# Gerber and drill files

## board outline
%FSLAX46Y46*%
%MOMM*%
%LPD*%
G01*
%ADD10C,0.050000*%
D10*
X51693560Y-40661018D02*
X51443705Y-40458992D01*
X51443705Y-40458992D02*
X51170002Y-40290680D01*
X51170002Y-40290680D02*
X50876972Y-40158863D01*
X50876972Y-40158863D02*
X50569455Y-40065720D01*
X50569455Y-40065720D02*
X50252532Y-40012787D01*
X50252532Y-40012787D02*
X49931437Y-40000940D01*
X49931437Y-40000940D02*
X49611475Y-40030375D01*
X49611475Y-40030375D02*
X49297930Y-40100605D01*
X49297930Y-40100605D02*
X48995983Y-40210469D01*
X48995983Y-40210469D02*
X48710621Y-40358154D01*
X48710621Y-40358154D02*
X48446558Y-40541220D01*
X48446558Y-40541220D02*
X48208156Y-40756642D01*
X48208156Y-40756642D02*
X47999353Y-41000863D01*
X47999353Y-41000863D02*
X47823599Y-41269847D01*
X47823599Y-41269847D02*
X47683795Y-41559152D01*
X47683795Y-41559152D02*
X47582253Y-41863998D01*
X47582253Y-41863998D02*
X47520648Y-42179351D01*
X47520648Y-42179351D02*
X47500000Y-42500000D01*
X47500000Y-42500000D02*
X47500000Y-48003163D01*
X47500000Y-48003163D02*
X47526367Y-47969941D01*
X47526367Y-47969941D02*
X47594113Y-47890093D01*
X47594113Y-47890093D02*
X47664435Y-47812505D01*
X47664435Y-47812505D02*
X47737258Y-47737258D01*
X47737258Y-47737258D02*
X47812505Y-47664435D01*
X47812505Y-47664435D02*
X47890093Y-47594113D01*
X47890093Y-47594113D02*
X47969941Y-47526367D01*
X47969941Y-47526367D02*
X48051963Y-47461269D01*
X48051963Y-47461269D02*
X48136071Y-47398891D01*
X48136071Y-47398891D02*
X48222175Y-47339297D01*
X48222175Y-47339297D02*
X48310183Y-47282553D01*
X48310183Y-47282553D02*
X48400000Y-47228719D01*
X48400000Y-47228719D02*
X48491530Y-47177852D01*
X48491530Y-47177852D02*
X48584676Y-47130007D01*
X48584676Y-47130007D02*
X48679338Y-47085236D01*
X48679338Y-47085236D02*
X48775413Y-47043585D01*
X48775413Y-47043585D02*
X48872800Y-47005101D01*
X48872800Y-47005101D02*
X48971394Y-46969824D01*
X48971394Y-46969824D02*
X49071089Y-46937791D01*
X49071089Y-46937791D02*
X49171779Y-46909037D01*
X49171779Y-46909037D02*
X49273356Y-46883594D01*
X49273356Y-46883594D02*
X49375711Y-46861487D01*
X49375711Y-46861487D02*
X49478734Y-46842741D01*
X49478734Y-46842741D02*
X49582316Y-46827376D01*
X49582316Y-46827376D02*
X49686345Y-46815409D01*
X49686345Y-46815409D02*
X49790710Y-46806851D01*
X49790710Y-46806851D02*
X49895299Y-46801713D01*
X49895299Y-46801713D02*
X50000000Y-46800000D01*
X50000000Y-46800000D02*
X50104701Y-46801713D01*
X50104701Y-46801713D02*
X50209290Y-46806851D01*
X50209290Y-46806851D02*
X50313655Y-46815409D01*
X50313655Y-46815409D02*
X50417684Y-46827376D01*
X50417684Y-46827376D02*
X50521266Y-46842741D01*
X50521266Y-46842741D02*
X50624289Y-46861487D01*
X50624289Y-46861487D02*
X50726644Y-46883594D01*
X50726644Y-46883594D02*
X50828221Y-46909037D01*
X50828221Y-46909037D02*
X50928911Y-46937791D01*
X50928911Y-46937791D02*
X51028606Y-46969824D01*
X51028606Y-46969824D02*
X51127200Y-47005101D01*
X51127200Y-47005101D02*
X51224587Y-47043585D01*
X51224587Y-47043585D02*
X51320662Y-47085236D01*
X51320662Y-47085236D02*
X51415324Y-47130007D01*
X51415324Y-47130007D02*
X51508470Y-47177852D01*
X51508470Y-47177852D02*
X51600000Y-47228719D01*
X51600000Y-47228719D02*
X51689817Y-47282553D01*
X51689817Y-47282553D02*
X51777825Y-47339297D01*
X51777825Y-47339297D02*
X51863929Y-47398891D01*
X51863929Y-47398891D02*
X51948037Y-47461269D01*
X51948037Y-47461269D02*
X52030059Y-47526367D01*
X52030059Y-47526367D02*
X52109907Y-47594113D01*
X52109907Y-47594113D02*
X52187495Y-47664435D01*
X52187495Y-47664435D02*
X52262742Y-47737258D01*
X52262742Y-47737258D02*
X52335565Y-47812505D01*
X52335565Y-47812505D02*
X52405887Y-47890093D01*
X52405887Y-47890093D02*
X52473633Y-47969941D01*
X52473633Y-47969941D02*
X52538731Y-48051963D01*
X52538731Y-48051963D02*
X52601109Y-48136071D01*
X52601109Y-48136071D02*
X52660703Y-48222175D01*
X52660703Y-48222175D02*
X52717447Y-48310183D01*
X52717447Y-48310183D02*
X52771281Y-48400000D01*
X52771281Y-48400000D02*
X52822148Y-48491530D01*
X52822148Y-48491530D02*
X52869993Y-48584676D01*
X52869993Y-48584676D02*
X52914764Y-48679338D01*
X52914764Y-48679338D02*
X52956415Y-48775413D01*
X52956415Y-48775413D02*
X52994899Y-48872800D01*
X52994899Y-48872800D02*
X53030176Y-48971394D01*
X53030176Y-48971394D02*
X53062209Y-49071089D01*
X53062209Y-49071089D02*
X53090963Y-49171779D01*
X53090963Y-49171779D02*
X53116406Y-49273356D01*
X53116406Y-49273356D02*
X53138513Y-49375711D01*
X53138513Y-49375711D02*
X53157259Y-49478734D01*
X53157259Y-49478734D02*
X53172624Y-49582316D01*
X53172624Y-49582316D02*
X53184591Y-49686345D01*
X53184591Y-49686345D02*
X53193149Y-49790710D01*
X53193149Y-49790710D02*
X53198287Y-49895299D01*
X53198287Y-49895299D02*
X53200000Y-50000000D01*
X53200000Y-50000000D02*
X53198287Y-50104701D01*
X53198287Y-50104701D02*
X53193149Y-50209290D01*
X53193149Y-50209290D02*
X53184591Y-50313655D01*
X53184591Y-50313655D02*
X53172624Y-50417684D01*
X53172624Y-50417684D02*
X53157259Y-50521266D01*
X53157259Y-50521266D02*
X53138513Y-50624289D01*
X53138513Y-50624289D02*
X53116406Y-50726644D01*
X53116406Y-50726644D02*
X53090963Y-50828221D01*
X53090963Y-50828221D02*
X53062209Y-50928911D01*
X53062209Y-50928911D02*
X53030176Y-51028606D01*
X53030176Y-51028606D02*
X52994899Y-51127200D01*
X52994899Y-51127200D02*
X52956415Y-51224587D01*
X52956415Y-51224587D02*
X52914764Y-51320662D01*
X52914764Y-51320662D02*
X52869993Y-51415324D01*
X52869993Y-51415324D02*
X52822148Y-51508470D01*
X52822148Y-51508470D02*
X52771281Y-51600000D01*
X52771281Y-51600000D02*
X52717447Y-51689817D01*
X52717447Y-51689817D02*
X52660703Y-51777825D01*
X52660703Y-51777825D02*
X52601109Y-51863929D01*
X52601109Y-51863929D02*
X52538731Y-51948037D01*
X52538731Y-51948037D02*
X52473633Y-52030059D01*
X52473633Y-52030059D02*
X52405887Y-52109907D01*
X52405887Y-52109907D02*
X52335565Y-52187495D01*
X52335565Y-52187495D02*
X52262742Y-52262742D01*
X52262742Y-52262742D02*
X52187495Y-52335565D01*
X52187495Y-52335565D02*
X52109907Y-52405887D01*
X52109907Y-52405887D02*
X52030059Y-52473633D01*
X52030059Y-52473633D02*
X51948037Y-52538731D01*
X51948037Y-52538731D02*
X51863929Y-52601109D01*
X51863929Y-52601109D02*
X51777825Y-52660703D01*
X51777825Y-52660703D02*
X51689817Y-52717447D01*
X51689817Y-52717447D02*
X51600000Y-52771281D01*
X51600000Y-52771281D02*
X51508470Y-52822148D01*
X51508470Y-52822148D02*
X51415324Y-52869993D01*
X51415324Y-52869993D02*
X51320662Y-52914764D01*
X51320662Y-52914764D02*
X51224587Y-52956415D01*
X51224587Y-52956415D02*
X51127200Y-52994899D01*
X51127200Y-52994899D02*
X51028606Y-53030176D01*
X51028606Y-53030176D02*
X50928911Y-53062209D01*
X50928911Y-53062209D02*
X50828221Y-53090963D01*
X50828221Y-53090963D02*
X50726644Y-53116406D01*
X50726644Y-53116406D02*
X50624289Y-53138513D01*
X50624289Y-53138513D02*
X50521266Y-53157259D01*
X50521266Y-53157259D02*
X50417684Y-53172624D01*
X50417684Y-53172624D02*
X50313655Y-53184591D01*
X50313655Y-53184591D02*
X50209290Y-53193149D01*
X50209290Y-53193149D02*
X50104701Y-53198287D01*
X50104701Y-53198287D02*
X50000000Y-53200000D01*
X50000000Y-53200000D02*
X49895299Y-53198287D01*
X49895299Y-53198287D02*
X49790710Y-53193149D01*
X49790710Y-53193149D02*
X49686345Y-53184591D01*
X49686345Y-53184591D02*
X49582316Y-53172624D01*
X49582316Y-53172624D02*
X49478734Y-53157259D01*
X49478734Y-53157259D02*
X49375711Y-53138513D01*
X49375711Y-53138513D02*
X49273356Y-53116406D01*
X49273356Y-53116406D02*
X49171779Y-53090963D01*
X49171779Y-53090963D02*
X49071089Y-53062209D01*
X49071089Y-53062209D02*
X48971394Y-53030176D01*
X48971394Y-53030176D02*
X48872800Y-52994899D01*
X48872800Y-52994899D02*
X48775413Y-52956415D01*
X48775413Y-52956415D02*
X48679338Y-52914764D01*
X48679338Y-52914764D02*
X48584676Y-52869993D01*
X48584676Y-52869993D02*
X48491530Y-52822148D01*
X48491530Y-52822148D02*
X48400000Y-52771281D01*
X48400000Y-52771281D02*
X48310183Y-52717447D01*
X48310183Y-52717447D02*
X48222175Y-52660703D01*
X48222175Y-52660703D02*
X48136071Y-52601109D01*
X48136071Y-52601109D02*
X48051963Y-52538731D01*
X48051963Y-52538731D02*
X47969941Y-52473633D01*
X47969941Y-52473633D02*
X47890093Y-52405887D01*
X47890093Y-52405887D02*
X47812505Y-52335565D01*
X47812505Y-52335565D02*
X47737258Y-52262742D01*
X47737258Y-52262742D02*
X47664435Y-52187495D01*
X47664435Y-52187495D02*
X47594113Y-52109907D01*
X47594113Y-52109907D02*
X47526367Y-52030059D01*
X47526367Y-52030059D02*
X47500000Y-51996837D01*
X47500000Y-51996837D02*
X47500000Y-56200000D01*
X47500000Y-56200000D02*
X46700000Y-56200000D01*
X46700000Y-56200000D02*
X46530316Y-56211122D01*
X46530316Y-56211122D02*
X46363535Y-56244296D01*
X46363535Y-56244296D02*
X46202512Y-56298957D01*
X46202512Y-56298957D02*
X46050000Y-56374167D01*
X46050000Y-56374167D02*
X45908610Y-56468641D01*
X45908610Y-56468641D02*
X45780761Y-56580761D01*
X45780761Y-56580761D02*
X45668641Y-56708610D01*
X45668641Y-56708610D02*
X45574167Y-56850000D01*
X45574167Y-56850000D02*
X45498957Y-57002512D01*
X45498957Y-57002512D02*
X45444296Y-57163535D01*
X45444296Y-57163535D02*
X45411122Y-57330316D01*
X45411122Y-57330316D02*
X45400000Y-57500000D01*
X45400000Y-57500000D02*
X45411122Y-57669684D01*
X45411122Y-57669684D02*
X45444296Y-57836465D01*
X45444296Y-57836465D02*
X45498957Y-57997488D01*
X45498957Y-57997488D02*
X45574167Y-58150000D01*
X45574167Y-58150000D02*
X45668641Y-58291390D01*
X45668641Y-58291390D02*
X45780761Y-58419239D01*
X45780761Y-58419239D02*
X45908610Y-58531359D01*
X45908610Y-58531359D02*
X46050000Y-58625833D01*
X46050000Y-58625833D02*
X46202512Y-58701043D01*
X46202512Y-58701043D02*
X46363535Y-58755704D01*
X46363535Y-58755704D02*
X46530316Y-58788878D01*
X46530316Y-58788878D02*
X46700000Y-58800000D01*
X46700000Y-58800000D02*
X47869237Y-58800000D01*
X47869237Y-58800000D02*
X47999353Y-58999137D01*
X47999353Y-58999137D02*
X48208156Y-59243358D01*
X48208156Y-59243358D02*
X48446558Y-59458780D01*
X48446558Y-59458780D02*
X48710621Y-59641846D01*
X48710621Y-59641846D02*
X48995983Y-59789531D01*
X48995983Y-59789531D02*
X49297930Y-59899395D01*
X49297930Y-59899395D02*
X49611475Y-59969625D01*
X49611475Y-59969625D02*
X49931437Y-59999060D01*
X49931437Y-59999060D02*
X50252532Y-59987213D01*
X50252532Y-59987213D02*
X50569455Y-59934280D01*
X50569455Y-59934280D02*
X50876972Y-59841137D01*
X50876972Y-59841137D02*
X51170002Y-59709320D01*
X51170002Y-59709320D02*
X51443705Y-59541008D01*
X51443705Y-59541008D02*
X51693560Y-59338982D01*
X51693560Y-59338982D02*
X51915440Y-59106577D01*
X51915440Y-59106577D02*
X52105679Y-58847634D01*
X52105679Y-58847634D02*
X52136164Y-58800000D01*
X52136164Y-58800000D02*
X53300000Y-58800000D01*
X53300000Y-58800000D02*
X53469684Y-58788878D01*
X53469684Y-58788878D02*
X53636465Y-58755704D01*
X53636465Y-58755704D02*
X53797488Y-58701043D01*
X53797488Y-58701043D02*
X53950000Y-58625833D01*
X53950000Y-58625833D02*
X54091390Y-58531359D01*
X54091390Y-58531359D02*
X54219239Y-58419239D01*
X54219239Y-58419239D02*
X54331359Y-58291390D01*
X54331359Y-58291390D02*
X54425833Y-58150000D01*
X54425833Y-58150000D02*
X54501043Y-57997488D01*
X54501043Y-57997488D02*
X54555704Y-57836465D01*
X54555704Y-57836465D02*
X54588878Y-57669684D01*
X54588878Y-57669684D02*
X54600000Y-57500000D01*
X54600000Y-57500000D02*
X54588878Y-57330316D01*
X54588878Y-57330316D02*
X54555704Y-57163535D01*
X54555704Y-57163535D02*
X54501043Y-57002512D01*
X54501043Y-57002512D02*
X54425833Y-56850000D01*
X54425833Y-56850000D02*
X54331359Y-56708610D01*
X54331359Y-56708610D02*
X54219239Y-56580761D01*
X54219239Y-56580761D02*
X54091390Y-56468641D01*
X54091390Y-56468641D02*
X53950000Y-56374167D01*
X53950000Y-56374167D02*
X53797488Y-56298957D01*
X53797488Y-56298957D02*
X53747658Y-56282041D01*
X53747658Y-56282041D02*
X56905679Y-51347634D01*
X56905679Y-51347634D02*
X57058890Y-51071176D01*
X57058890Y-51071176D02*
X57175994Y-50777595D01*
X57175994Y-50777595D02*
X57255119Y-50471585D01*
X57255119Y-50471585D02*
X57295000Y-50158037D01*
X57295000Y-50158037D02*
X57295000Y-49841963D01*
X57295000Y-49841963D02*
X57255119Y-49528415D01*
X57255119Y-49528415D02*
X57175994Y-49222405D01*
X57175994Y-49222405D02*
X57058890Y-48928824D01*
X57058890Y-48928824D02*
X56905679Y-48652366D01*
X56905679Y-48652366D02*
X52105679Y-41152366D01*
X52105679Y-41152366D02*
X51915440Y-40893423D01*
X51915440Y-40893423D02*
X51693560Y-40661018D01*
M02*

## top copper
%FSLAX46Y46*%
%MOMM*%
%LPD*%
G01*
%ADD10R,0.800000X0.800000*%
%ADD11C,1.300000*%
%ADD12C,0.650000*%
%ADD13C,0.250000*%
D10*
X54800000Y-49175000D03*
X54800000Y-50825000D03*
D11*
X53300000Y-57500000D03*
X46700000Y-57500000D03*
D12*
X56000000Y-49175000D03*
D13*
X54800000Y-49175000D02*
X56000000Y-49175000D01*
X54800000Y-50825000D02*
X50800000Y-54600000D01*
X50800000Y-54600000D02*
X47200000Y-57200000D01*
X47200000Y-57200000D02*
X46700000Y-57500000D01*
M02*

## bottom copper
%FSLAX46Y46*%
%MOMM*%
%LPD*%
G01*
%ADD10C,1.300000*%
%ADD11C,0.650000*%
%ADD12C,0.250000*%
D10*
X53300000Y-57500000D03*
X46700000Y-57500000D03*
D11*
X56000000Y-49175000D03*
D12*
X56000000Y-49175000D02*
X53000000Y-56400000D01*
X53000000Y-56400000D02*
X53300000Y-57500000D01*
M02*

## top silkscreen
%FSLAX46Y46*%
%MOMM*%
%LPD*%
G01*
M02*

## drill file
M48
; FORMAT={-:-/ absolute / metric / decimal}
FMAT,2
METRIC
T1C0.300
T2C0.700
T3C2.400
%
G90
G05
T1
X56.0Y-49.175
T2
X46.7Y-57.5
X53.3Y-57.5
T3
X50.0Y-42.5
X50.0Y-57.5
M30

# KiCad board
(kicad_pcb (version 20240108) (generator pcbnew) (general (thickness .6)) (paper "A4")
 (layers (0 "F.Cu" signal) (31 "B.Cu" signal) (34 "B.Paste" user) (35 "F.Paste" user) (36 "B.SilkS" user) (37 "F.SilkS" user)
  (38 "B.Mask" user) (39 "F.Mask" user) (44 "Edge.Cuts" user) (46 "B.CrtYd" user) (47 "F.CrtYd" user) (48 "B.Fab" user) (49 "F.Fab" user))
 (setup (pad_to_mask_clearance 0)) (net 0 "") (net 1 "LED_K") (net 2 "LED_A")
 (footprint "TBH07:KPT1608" (layer "F.Cu") (at 54.8 50)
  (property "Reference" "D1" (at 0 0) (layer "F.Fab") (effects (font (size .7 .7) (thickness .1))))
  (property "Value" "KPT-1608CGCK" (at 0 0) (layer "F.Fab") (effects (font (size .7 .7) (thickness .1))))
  (pad "1" smd rect (at 0 -.825) (size .8 .8) (layers "F.Cu" "F.Paste" "F.Mask") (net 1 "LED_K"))
  (pad "2" smd rect (at 0 .825) (size .8 .8) (layers "F.Cu" "F.Paste" "F.Mask") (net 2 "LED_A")))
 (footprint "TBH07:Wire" (layer "F.Cu") (at 53.3 57.5)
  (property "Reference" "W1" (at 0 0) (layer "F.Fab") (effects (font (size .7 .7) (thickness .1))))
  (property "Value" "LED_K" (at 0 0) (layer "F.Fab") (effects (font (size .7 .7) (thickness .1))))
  (pad "1" thru_hole circle (at 0 0) (size 1.3 1.3) (drill .7) (layers "*.Cu" "*.Mask") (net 1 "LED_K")))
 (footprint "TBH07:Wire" (layer "F.Cu") (at 46.7 57.5)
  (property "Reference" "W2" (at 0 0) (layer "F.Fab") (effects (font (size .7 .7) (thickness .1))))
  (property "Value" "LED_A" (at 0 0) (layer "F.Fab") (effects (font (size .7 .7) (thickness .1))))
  (pad "1" thru_hole circle (at 0 0) (size 1.3 1.3) (drill .7) (layers "*.Cu" "*.Mask") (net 2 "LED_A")))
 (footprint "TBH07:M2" (layer "F.Cu") (at 50 42.5)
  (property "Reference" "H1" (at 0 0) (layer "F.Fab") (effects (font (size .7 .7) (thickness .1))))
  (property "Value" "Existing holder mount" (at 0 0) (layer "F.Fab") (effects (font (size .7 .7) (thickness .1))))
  (pad "" np_thru_hole circle (at 0 0) (size 2.4 2.4) (drill 2.4) (layers "*.Cu" "*.Mask")))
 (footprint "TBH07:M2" (layer "F.Cu") (at 50 57.5)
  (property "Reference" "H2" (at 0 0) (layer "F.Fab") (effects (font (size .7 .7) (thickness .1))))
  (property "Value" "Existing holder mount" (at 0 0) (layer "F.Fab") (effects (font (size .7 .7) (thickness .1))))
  (pad "" np_thru_hole circle (at 0 0) (size 2.4 2.4) (drill 2.4) (layers "*.Cu" "*.Mask")))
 (segment (start 54.8 49.175) (end 56 49.175) (width .25) (layer "F.Cu") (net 1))
 (via (at 56 49.175) (size .65) (drill .3) (layers "F.Cu" "B.Cu") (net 1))
 (segment (start 56 49.175) (end 53.0 56.4) (width .25) (layer "B.Cu") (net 1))
 (segment (start 53.0 56.4) (end 53.3 57.5) (width .25) (layer "B.Cu") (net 1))
 (segment (start 54.8 50.825) (end 50.8 54.6) (width .25) (layer "F.Cu") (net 2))
 (segment (start 50.8 54.6) (end 47.2 57.2) (width .25) (layer "F.Cu") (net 2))
 (segment (start 47.2 57.2) (end 46.7 57.5) (width .25) (layer "F.Cu") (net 2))
 (gr_line (start 51.69356030307014 40.661018352493706) (end 51.443705330258624 40.45899169051597) (stroke (width .05) (type default))
  (layer "Edge.Cuts"))
 (gr_line (start 51.443705330258624 40.45899169051597) (end 51.170002128751115 40.29067996462308) (stroke (width .05) (type default))
  (layer "Edge.Cuts"))
 (gr_line (start 51.170002128751115 40.29067996462308) (end 50.8769719373403 40.15886347661705) (stroke (width .05) (type default))
  (layer "Edge.Cuts"))
 (gr_line (start 50.8769719373403 40.15886347661705) (end 50.569455252818095 40.06571967205133) (stroke (width .05) (type default))
  (layer "Edge.Cuts"))
 (gr_line (start 50.569455252818095 40.06571967205133) (end 50.25253187094796 40.01278717151999) (stroke (width .05) (type default))
  (layer "Edge.Cuts"))
 (gr_line (start 50.25253187094796 40.01278717151999) (end 49.93143697451376 40.0009403545461) (stroke (width .05) (type default))
  (layer "Edge.Cuts"))
 (gr_line (start 49.93143697451376 40.0009403545461) (end 49.61147465456702 40.0303749159121) (stroke (width .05) (type default))
  (layer "Edge.Cuts"))
 (gr_line (start 49.61147465456702 40.0303749159121) (end 49.29793029339476 40.10060463302372) (stroke (width .05) (type default))
  (layer "Edge.Cuts"))
 (gr_line (start 49.29793029339476 40.10060463302372) (end 48.995983256532874 40.21046939770667) (stroke (width .05) (type default))
  (layer "Edge.Cuts"))
 (gr_line (start 48.995983256532874 40.21046939770667) (end 48.71062133604549 40.358154379760556) (stroke (width .05) (type default))
  (layer "Edge.Cuts"))
 (gr_line (start 48.71062133604549 40.358154379760556) (end 48.44655835836122 40.54122000571207) (stroke (width .05) (type default))
  (layer "Edge.Cuts"))
 (gr_line (start 48.44655835836122 40.54122000571207) (end 48.20815631768343 40.756642257555214) (stroke (width .05) (type default))
  (layer "Edge.Cuts"))
 (gr_line (start 48.20815631768343 40.756642257555214) (end 47.99935332123422 41.000862625793275) (stroke (width .05) (type default))
  (layer "Edge.Cuts"))
 (gr_line (start 47.99935332123422 41.000862625793275) (end 47.82359853658772 41.26984689162005) (stroke (width .05) (type default))
  (layer "Edge.Cuts"))
 (gr_line (start 47.82359853658772 41.26984689162005) (end 47.68379521568241 41.55915176723114) (stroke (width .05) (type default))
  (layer "Edge.Cuts"))
 (gr_line (start 47.68379521568241 41.55915176723114) (end 47.582252736685376 41.863998293449896) (stroke (width .05) (type default))
  (layer "Edge.Cuts"))
 (gr_line (start 47.582252736685376 41.863998293449896) (end 47.5206484559177 42.179350782229676) (stroke (width .05) (type default))
  (layer "Edge.Cuts"))
 (gr_line (start 47.5206484559177 42.179350782229676) (end 47.5 42.5) (stroke (width .05) (type default)) (layer "Edge.Cuts"))
 (gr_line (start 47.5 42.5) (end 47.5 48.00316310634037) (stroke (width .05) (type default)) (layer "Edge.Cuts"))
 (gr_line (start 47.5 48.00316310634037) (end 47.52636654923924 47.969941490676334) (stroke (width .05) (type default)) (layer "Edge.Cuts"))
 (gr_line (start 47.52636654923924 47.969941490676334) (end 47.59411261606727 47.89009339167978) (stroke (width .05) (type default))
  (layer "Edge.Cuts"))
 (gr_line (start 47.59411261606727 47.89009339167978) (end 47.66443496736693 47.812504633526814) (stroke (width .05) (type default))
  (layer "Edge.Cuts"))
 (gr_line (start 47.66443496736693 47.812504633526814) (end 47.737258300203045 47.737258300203045) (stroke (width .05) (type default))
  (layer "Edge.Cuts"))
 (gr_line (start 47.737258300203045 47.737258300203045) (end 47.812504633526814 47.66443496736692) (stroke (width .05) (type default))
  (layer "Edge.Cuts"))
 (gr_line (start 47.812504633526814 47.66443496736692) (end 47.890093391679784 47.59411261606727) (stroke (width .05) (type default))
  (layer "Edge.Cuts"))
 (gr_line (start 47.890093391679784 47.59411261606727) (end 47.969941490676334 47.52636654923924) (stroke (width .05) (type default))
  (layer "Edge.Cuts"))
 (gr_line (start 47.969941490676334 47.52636654923924) (end 48.0519634271721 47.461269311068044) (stroke (width .05) (type default))
  (layer "Edge.Cuts"))
 (gr_line (start 48.0519634271721 47.461269311068044) (end 48.13607137002303 47.39889060930683) (stroke (width .05) (type default))
  (layer "Edge.Cuts"))
 (gr_line (start 48.13607137002303 47.39889060930683) (end 48.22217525433727 47.33929724063186) (stroke (width .05) (type default))
  (layer "Edge.Cuts"))
 (gr_line (start 48.22217525433727 47.33929724063186) (end 48.31018287791882 47.28255301911495) (stroke (width .05) (type default))
  (layer "Edge.Cuts"))
 (gr_line (start 48.31018287791882 47.28255301911495) (end 48.4 47.2287187078898) (stroke (width .05) (type default)) (layer "Edge.Cuts"))
 (gr_line (start 48.4 47.2287187078898) (end 48.49153044215681 47.17785195408526) (stroke (width .05) (type default)) (layer "Edge.Cuts"))
 (gr_line (start 48.49153044215681 47.17785195408526) (end 48.584676191299195 47.1300072270954) (stroke (width .05) (type default))
  (layer "Edge.Cuts"))
 (gr_line (start 48.584676191299195 47.1300072270954) (end 48.679337504625934 47.08523576025224) (stroke (width .05) (type default))
  (layer "Edge.Cuts"))
 (gr_line (start 48.679337504625934 47.08523576025224) (end 48.77541301643171 47.04358549596388) (stroke (width .05) (type default))
  (layer "Edge.Cuts"))
 (gr_line (start 48.77541301643171 47.04358549596388) (end 48.87279984665205 47.00510103437656) (stroke (width .05) (type default))
  (layer "Edge.Cuts"))
 (gr_line (start 48.87279984665205 47.00510103437656) (end 48.97139371102988 46.969823585615664) (stroke (width .05) (type default))
  (layer "Edge.Cuts"))
 (gr_line (start 48.97139371102988 46.969823585615664) (end 49.07108903278572 46.937790925656934) (stroke (width .05) (type default))
  (layer "Edge.Cuts"))
 (gr_line (start 49.07108903278572 46.937790925656934) (end 49.171779055671934 46.90903735587498) (stroke (width .05) (type default))
  (layer "Edge.Cuts"))
 (gr_line (start 49.171779055671934 46.90903735587498) (end 49.273355958290004 46.883593666312535) (stroke (width .05) (type default))
  (layer "Edge.Cuts"))
 (gr_line (start 49.273355958290004 46.883593666312535) (end 49.37571096954839 46.86148710270966) (stroke (width .05) (type default))
  (layer "Edge.Cuts"))
 (gr_line (start 49.37571096954839 46.86148710270966) (end 49.478734485137316 46.842741337328384) (stroke (width .05) (type default))
  (layer "Edge.Cuts"))
 (gr_line (start 49.478734485137316 46.842741337328384) (end 49.58231618489584 46.827376443603804) (stroke (width .05) (type default))
  (layer "Edge.Cuts"))
 (gr_line (start 49.58231618489584 46.827376443603804) (end 49.68634515094541 46.815408874648966) (stroke (width .05) (type default))
  (layer "Edge.Cuts"))
 (gr_line (start 49.68634515094541 46.815408874648966) (end 49.79070998646354 46.80685144563647) (stroke (width .05) (type default))
  (layer "Edge.Cuts"))
 (gr_line (start 49.79070998646354 46.80685144563647) (end 49.89529893497032 46.80171332007563) (stroke (width .05) (type default))
  (layer "Edge.Cuts"))
 (gr_line (start 49.89529893497032 46.80171332007563) (end 50.0 46.8) (stroke (width .05) (type default)) (layer "Edge.Cuts"))
 (gr_line (start 50.0 46.8) (end 50.10470106502969 46.80171332007563) (stroke (width .05) (type default)) (layer "Edge.Cuts"))
 (gr_line (start 50.10470106502969 46.80171332007563) (end 50.20929001353646 46.80685144563647) (stroke (width .05) (type default))
  (layer "Edge.Cuts"))
 (gr_line (start 50.20929001353646 46.80685144563647) (end 50.31365484905459 46.815408874648966) (stroke (width .05) (type default))
  (layer "Edge.Cuts"))
 (gr_line (start 50.31365484905459 46.815408874648966) (end 50.41768381510416 46.827376443603804) (stroke (width .05) (type default))
  (layer "Edge.Cuts"))
 (gr_line (start 50.41768381510416 46.827376443603804) (end 50.521265514862684 46.842741337328384) (stroke (width .05) (type default))
  (layer "Edge.Cuts"))
 (gr_line (start 50.521265514862684 46.842741337328384) (end 50.624289030451614 46.86148710270966) (stroke (width .05) (type default))
  (layer "Edge.Cuts"))
 (gr_line (start 50.624289030451614 46.86148710270966) (end 50.726644041709996 46.883593666312535) (stroke (width .05) (type default))
  (layer "Edge.Cuts"))
 (gr_line (start 50.726644041709996 46.883593666312535) (end 50.828220944328066 46.90903735587498) (stroke (width .05) (type default))
  (layer "Edge.Cuts"))
 (gr_line (start 50.828220944328066 46.90903735587498) (end 50.92891096721428 46.937790925656934) (stroke (width .05) (type default))
  (layer "Edge.Cuts"))
 (gr_line (start 50.92891096721428 46.937790925656934) (end 51.02860628897012 46.969823585615664) (stroke (width .05) (type default))
  (layer "Edge.Cuts"))
 (gr_line (start 51.02860628897012 46.969823585615664) (end 51.12720015334795 47.00510103437656) (stroke (width .05) (type default))
  (layer "Edge.Cuts"))
 (gr_line (start 51.12720015334795 47.00510103437656) (end 51.22458698356829 47.04358549596388) (stroke (width .05) (type default))
  (layer "Edge.Cuts"))
 (gr_line (start 51.22458698356829 47.04358549596388) (end 51.320662495374066 47.08523576025224) (stroke (width .05) (type default))
  (layer "Edge.Cuts"))
 (gr_line (start 51.320662495374066 47.08523576025224) (end 51.415323808700805 47.1300072270954) (stroke (width .05) (type default))
  (layer "Edge.Cuts"))
 (gr_line (start 51.415323808700805 47.1300072270954) (end 51.50846955784319 47.17785195408526) (stroke (width .05) (type default))
  (layer "Edge.Cuts"))
 (gr_line (start 51.50846955784319 47.17785195408526) (end 51.6 47.2287187078898) (stroke (width .05) (type default)) (layer "Edge.Cuts"))
 (gr_line (start 51.6 47.2287187078898) (end 51.68981712208118 47.28255301911495) (stroke (width .05) (type default)) (layer "Edge.Cuts"))
 (gr_line (start 51.68981712208118 47.28255301911495) (end 51.77782474566273 47.33929724063186) (stroke (width .05) (type default))
  (layer "Edge.Cuts"))
 (gr_line (start 51.77782474566273 47.33929724063186) (end 51.86392862997697 47.39889060930683) (stroke (width .05) (type default))
  (layer "Edge.Cuts"))
 (gr_line (start 51.86392862997697 47.39889060930683) (end 51.9480365728279 47.46126931106805) (stroke (width .05) (type default))
  (layer "Edge.Cuts"))
 (gr_line (start 51.9480365728279 47.46126931106805) (end 52.030058509323666 47.52636654923924) (stroke (width .05) (type default))
  (layer "Edge.Cuts"))
 (gr_line (start 52.030058509323666 47.52636654923924) (end 52.10990660832022 47.59411261606727) (stroke (width .05) (type default))
  (layer "Edge.Cuts"))
 (gr_line (start 52.10990660832022 47.59411261606727) (end 52.187495366473186 47.66443496736693) (stroke (width .05) (type default))
  (layer "Edge.Cuts"))
 (gr_line (start 52.187495366473186 47.66443496736693) (end 52.262741699796955 47.737258300203045) (stroke (width .05) (type default))
  (layer "Edge.Cuts"))
 (gr_line (start 52.262741699796955 47.737258300203045) (end 52.33556503263308 47.812504633526814) (stroke (width .05) (type default))
  (layer "Edge.Cuts"))
 (gr_line (start 52.33556503263308 47.812504633526814) (end 52.40588738393273 47.89009339167978) (stroke (width .05) (type default))
  (layer "Edge.Cuts"))
 (gr_line (start 52.40588738393273 47.89009339167978) (end 52.47363345076076 47.969941490676334) (stroke (width .05) (type default))
  (layer "Edge.Cuts"))
 (gr_line (start 52.47363345076076 47.969941490676334) (end 52.538730688931956 48.0519634271721) (stroke (width .05) (type default))
  (layer "Edge.Cuts"))
 (gr_line (start 52.538730688931956 48.0519634271721) (end 52.60110939069317 48.13607137002303) (stroke (width .05) (type default))
  (layer "Edge.Cuts"))
 (gr_line (start 52.60110939069317 48.13607137002303) (end 52.66070275936814 48.22217525433727) (stroke (width .05) (type default))
  (layer "Edge.Cuts"))
 (gr_line (start 52.66070275936814 48.22217525433727) (end 52.71744698088505 48.31018287791882) (stroke (width .05) (type default))
  (layer "Edge.Cuts"))
 (gr_line (start 52.71744698088505 48.31018287791882) (end 52.7712812921102 48.4) (stroke (width .05) (type default)) (layer "Edge.Cuts"))
 (gr_line (start 52.7712812921102 48.4) (end 52.82214804591474 48.49153044215681) (stroke (width .05) (type default)) (layer "Edge.Cuts"))
 (gr_line (start 52.82214804591474 48.49153044215681) (end 52.8699927729046 48.584676191299195) (stroke (width .05) (type default))
  (layer "Edge.Cuts"))
 (gr_line (start 52.8699927729046 48.584676191299195) (end 52.91476423974776 48.679337504625934) (stroke (width .05) (type default))
  (layer "Edge.Cuts"))
 (gr_line (start 52.91476423974776 48.679337504625934) (end 52.95641450403612 48.77541301643171) (stroke (width .05) (type default))
  (layer "Edge.Cuts"))
 (gr_line (start 52.95641450403612 48.77541301643171) (end 52.99489896562344 48.87279984665205) (stroke (width .05) (type default))
  (layer "Edge.Cuts"))
 (gr_line (start 52.99489896562344 48.87279984665205) (end 53.030176414384336 48.97139371102988) (stroke (width .05) (type default))
  (layer "Edge.Cuts"))
 (gr_line (start 53.030176414384336 48.97139371102988) (end 53.062209074343066 49.07108903278572) (stroke (width .05) (type default))
  (layer "Edge.Cuts"))
 (gr_line (start 53.062209074343066 49.07108903278572) (end 53.09096264412502 49.171779055671934) (stroke (width .05) (type default))
  (layer "Edge.Cuts"))
 (gr_line (start 53.09096264412502 49.171779055671934) (end 53.116406333687465 49.273355958290004) (stroke (width .05) (type default))
  (layer "Edge.Cuts"))
 (gr_line (start 53.116406333687465 49.273355958290004) (end 53.13851289729034 49.375710969548386) (stroke (width .05) (type default))
  (layer "Edge.Cuts"))
 (gr_line (start 53.13851289729034 49.375710969548386) (end 53.157258662671616 49.478734485137316) (stroke (width .05) (type default))
  (layer "Edge.Cuts"))
 (gr_line (start 53.157258662671616 49.478734485137316) (end 53.172623556396196 49.58231618489584) (stroke (width .05) (type default))
  (layer "Edge.Cuts"))
 (gr_line (start 53.172623556396196 49.58231618489584) (end 53.184591125351034 49.68634515094541) (stroke (width .05) (type default))
  (layer "Edge.Cuts"))
 (gr_line (start 53.184591125351034 49.68634515094541) (end 53.19314855436353 49.79070998646354) (stroke (width .05) (type default))
  (layer "Edge.Cuts"))
 (gr_line (start 53.19314855436353 49.79070998646354) (end 53.19828667992437 49.89529893497031) (stroke (width .05) (type default))
  (layer "Edge.Cuts"))
 (gr_line (start 53.19828667992437 49.89529893497031) (end 53.2 50.0) (stroke (width .05) (type default)) (layer "Edge.Cuts"))
 (gr_line (start 53.2 50.0) (end 53.19828667992437 50.10470106502969) (stroke (width .05) (type default)) (layer "Edge.Cuts"))
 (gr_line (start 53.19828667992437 50.10470106502969) (end 53.19314855436353 50.20929001353646) (stroke (width .05) (type default))
  (layer "Edge.Cuts"))
 (gr_line (start 53.19314855436353 50.20929001353646) (end 53.184591125351034 50.31365484905459) (stroke (width .05) (type default))
  (layer "Edge.Cuts"))
 (gr_line (start 53.184591125351034 50.31365484905459) (end 53.17262355639619 50.41768381510417) (stroke (width .05) (type default))
  (layer "Edge.Cuts"))
 (gr_line (start 53.17262355639619 50.41768381510417) (end 53.157258662671616 50.521265514862684) (stroke (width .05) (type default))
  (layer "Edge.Cuts"))
 (gr_line (start 53.157258662671616 50.521265514862684) (end 53.13851289729034 50.624289030451614) (stroke (width .05) (type default))
  (layer "Edge.Cuts"))
 (gr_line (start 53.13851289729034 50.624289030451614) (end 53.116406333687465 50.726644041709996) (stroke (width .05) (type default))
  (layer "Edge.Cuts"))
 (gr_line (start 53.116406333687465 50.726644041709996) (end 53.09096264412502 50.828220944328066) (stroke (width .05) (type default))
  (layer "Edge.Cuts"))
 (gr_line (start 53.09096264412502 50.828220944328066) (end 53.062209074343066 50.928910967214286) (stroke (width .05) (type default))
  (layer "Edge.Cuts"))
 (gr_line (start 53.062209074343066 50.928910967214286) (end 53.030176414384336 51.02860628897012) (stroke (width .05) (type default))
  (layer "Edge.Cuts"))
 (gr_line (start 53.030176414384336 51.02860628897012) (end 52.99489896562344 51.12720015334795) (stroke (width .05) (type default))
  (layer "Edge.Cuts"))
 (gr_line (start 52.99489896562344 51.12720015334795) (end 52.95641450403612 51.22458698356829) (stroke (width .05) (type default))
  (layer "Edge.Cuts"))
 (gr_line (start 52.95641450403612 51.22458698356829) (end 52.91476423974776 51.320662495374066) (stroke (width .05) (type default))
  (layer "Edge.Cuts"))
 (gr_line (start 52.91476423974776 51.320662495374066) (end 52.8699927729046 51.415323808700805) (stroke (width .05) (type default))
  (layer "Edge.Cuts"))
 (gr_line (start 52.8699927729046 51.415323808700805) (end 52.82214804591474 51.50846955784319) (stroke (width .05) (type default))
  (layer "Edge.Cuts"))
 (gr_line (start 52.82214804591474 51.50846955784319) (end 52.7712812921102 51.6) (stroke (width .05) (type default)) (layer "Edge.Cuts"))
 (gr_line (start 52.7712812921102 51.6) (end 52.71744698088505 51.68981712208118) (stroke (width .05) (type default)) (layer "Edge.Cuts"))
 (gr_line (start 52.71744698088505 51.68981712208118) (end 52.66070275936814 51.77782474566273) (stroke (width .05) (type default))
  (layer "Edge.Cuts"))
 (gr_line (start 52.66070275936814 51.77782474566273) (end 52.60110939069317 51.86392862997697) (stroke (width .05) (type default))
  (layer "Edge.Cuts"))
 (gr_line (start 52.60110939069317 51.86392862997697) (end 52.53873068893195 51.94803657282791) (stroke (width .05) (type default))
  (layer "Edge.Cuts"))
 (gr_line (start 52.53873068893195 51.94803657282791) (end 52.47363345076076 52.030058509323666) (stroke (width .05) (type default))
  (layer "Edge.Cuts"))
 (gr_line (start 52.47363345076076 52.030058509323666) (end 52.40588738393273 52.10990660832022) (stroke (width .05) (type default))
  (layer "Edge.Cuts"))
 (gr_line (start 52.40588738393273 52.10990660832022) (end 52.33556503263307 52.18749536647319) (stroke (width .05) (type default))
  (layer "Edge.Cuts"))
 (gr_line (start 52.33556503263307 52.18749536647319) (end 52.262741699796955 52.262741699796955) (stroke (width .05) (type default))
  (layer "Edge.Cuts"))
 (gr_line (start 52.262741699796955 52.262741699796955) (end 52.187495366473186 52.33556503263308) (stroke (width .05) (type default))
  (layer "Edge.Cuts"))
 (gr_line (start 52.187495366473186 52.33556503263308) (end 52.109906608320216 52.40588738393273) (stroke (width .05) (type default))
  (layer "Edge.Cuts"))
 (gr_line (start 52.109906608320216 52.40588738393273) (end 52.030058509323666 52.47363345076076) (stroke (width .05) (type default))
  (layer "Edge.Cuts"))
 (gr_line (start 52.030058509323666 52.47363345076076) (end 51.9480365728279 52.538730688931956) (stroke (width .05) (type default))
  (layer "Edge.Cuts"))
 (gr_line (start 51.9480365728279 52.538730688931956) (end 51.86392862997697 52.60110939069317) (stroke (width .05) (type default))
  (layer "Edge.Cuts"))
 (gr_line (start 51.86392862997697 52.60110939069317) (end 51.77782474566273 52.66070275936815) (stroke (width .05) (type default))
  (layer "Edge.Cuts"))
 (gr_line (start 51.77782474566273 52.66070275936815) (end 51.68981712208117 52.71744698088506) (stroke (width .05) (type default))
  (layer "Edge.Cuts"))
 (gr_line (start 51.68981712208117 52.71744698088506) (end 51.599999999999994 52.7712812921102) (stroke (width .05) (type default))
  (layer "Edge.Cuts"))
 (gr_line (start 51.599999999999994 52.7712812921102) (end 51.50846955784319 52.82214804591474) (stroke (width .05) (type default))
  (layer "Edge.Cuts"))
 (gr_line (start 51.50846955784319 52.82214804591474) (end 51.415323808700805 52.8699927729046) (stroke (width .05) (type default))
  (layer "Edge.Cuts"))
 (gr_line (start 51.415323808700805 52.8699927729046) (end 51.32066249537406 52.91476423974776) (stroke (width .05) (type default))
  (layer "Edge.Cuts"))
 (gr_line (start 51.32066249537406 52.91476423974776) (end 51.22458698356829 52.95641450403612) (stroke (width .05) (type default))
  (layer "Edge.Cuts"))
 (gr_line (start 51.22458698356829 52.95641450403612) (end 51.12720015334794 52.99489896562344) (stroke (width .05) (type default))
  (layer "Edge.Cuts"))
 (gr_line (start 51.12720015334794 52.99489896562344) (end 51.02860628897012 53.030176414384336) (stroke (width .05) (type default))
  (layer "Edge.Cuts"))
 (gr_line (start 51.02860628897012 53.030176414384336) (end 50.92891096721428 53.062209074343066) (stroke (width .05) (type default))
  (layer "Edge.Cuts"))
 (gr_line (start 50.92891096721428 53.062209074343066) (end 50.828220944328066 53.09096264412502) (stroke (width .05) (type default))
  (layer "Edge.Cuts"))
 (gr_line (start 50.828220944328066 53.09096264412502) (end 50.72664404170999 53.116406333687465) (stroke (width .05) (type default))
  (layer "Edge.Cuts"))
 (gr_line (start 50.72664404170999 53.116406333687465) (end 50.62428903045161 53.13851289729034) (stroke (width .05) (type default))
  (layer "Edge.Cuts"))
 (gr_line (start 50.62428903045161 53.13851289729034) (end 50.521265514862684 53.157258662671616) (stroke (width .05) (type default))
  (layer "Edge.Cuts"))
 (gr_line (start 50.521265514862684 53.157258662671616) (end 50.41768381510416 53.172623556396196) (stroke (width .05) (type default))
  (layer "Edge.Cuts"))
 (gr_line (start 50.41768381510416 53.172623556396196) (end 50.31365484905459 53.184591125351034) (stroke (width .05) (type default))
  (layer "Edge.Cuts"))
 (gr_line (start 50.31365484905459 53.184591125351034) (end 50.20929001353645 53.19314855436353) (stroke (width .05) (type default))
  (layer "Edge.Cuts"))
 (gr_line (start 50.20929001353645 53.19314855436353) (end 50.10470106502968 53.19828667992437) (stroke (width .05) (type default))
  (layer "Edge.Cuts"))
 (gr_line (start 50.10470106502968 53.19828667992437) (end 50.0 53.2) (stroke (width .05) (type default)) (layer "Edge.Cuts"))
 (gr_line (start 50.0 53.2) (end 49.89529893497031 53.19828667992437) (stroke (width .05) (type default)) (layer "Edge.Cuts"))
 (gr_line (start 49.89529893497031 53.19828667992437) (end 49.79070998646354 53.19314855436353) (stroke (width .05) (type default))
  (layer "Edge.Cuts"))
 (gr_line (start 49.79070998646354 53.19314855436353) (end 49.68634515094541 53.184591125351034) (stroke (width .05) (type default))
  (layer "Edge.Cuts"))
 (gr_line (start 49.68634515094541 53.184591125351034) (end 49.58231618489583 53.17262355639619) (stroke (width .05) (type default))
  (layer "Edge.Cuts"))
 (gr_line (start 49.58231618489583 53.17262355639619) (end 49.478734485137316 53.157258662671616) (stroke (width .05) (type default))
  (layer "Edge.Cuts"))
 (gr_line (start 49.478734485137316 53.157258662671616) (end 49.375710969548386 53.13851289729034) (stroke (width .05) (type default))
  (layer "Edge.Cuts"))
 (gr_line (start 49.375710969548386 53.13851289729034) (end 49.273355958290004 53.116406333687465) (stroke (width .05) (type default))
  (layer "Edge.Cuts"))
 (gr_line (start 49.273355958290004 53.116406333687465) (end 49.171779055671934 53.09096264412502) (stroke (width .05) (type default))
  (layer "Edge.Cuts"))
 (gr_line (start 49.171779055671934 53.09096264412502) (end 49.07108903278572 53.062209074343066) (stroke (width .05) (type default))
  (layer "Edge.Cuts"))
 (gr_line (start 49.07108903278572 53.062209074343066) (end 48.97139371102988 53.030176414384336) (stroke (width .05) (type default))
  (layer "Edge.Cuts"))
 (gr_line (start 48.97139371102988 53.030176414384336) (end 48.87279984665205 52.99489896562344) (stroke (width .05) (type default))
  (layer "Edge.Cuts"))
 (gr_line (start 48.87279984665205 52.99489896562344) (end 48.77541301643171 52.95641450403612) (stroke (width .05) (type default))
  (layer "Edge.Cuts"))
 (gr_line (start 48.77541301643171 52.95641450403612) (end 48.679337504625934 52.91476423974776) (stroke (width .05) (type default))
  (layer "Edge.Cuts"))
 (gr_line (start 48.679337504625934 52.91476423974776) (end 48.584676191299195 52.8699927729046) (stroke (width .05) (type default))
  (layer "Edge.Cuts"))
 (gr_line (start 48.584676191299195 52.8699927729046) (end 48.49153044215681 52.82214804591474) (stroke (width .05) (type default))
  (layer "Edge.Cuts"))
 (gr_line (start 48.49153044215681 52.82214804591474) (end 48.4 52.7712812921102) (stroke (width .05) (type default)) (layer "Edge.Cuts"))
 (gr_line (start 48.4 52.7712812921102) (end 48.31018287791882 52.71744698088505) (stroke (width .05) (type default)) (layer "Edge.Cuts"))
 (gr_line (start 48.31018287791882 52.71744698088505) (end 48.22217525433727 52.66070275936814) (stroke (width .05) (type default))
  (layer "Edge.Cuts"))
 (gr_line (start 48.22217525433727 52.66070275936814) (end 48.13607137002303 52.60110939069317) (stroke (width .05) (type default))
  (layer "Edge.Cuts"))
 (gr_line (start 48.13607137002303 52.60110939069317) (end 48.05196342717209 52.53873068893195) (stroke (width .05) (type default))
  (layer "Edge.Cuts"))
 (gr_line (start 48.05196342717209 52.53873068893195) (end 47.969941490676334 52.47363345076076) (stroke (width .05) (type default))
  (layer "Edge.Cuts"))
 (gr_line (start 47.969941490676334 52.47363345076076) (end 47.89009339167978 52.40588738393273) (stroke (width .05) (type default))
  (layer "Edge.Cuts"))
 (gr_line (start 47.89009339167978 52.40588738393273) (end 47.812504633526814 52.33556503263307) (stroke (width .05) (type default))
  (layer "Edge.Cuts"))
 (gr_line (start 47.812504633526814 52.33556503263307) (end 47.737258300203045 52.26274169979695) (stroke (width .05) (type default))
  (layer "Edge.Cuts"))
 (gr_line (start 47.737258300203045 52.26274169979695) (end 47.66443496736692 52.187495366473186) (stroke (width .05) (type default))
  (layer "Edge.Cuts"))
 (gr_line (start 47.66443496736692 52.187495366473186) (end 47.59411261606727 52.109906608320216) (stroke (width .05) (type default))
  (layer "Edge.Cuts"))
 (gr_line (start 47.59411261606727 52.109906608320216) (end 47.52636654923924 52.030058509323666) (stroke (width .05) (type default))
  (layer "Edge.Cuts"))
 (gr_line (start 47.52636654923924 52.030058509323666) (end 47.5 51.99683689365963) (stroke (width .05) (type default)) (layer "Edge.Cuts"))
 (gr_line (start 47.5 51.99683689365963) (end 47.5 56.2) (stroke (width .05) (type default)) (layer "Edge.Cuts"))
 (gr_line (start 47.5 56.2) (end 46.7 56.2) (stroke (width .05) (type default)) (layer "Edge.Cuts"))
 (gr_line (start 46.7 56.2) (end 46.53031595011393 56.21112168021405) (stroke (width .05) (type default)) (layer "Edge.Cuts"))
 (gr_line (start 46.53031595011393 56.21112168021405) (end 46.363535241366726 56.24429642582421) (stroke (width .05) (type default))
  (layer "Edge.Cuts"))
 (gr_line (start 46.363535241366726 56.24429642582421) (end 46.20251153792538 56.29895660773533) (stroke (width .05) (type default))
  (layer "Edge.Cuts"))
 (gr_line (start 46.20251153792538 56.29895660773533) (end 46.05 56.37416697508023) (stroke (width .05) (type default)) (layer "Edge.Cuts"))
 (gr_line (start 46.05 56.37416697508023) (end 45.908610142288666 56.46864065762139) (stroke (width .05) (type default)) (layer "Edge.Cuts"))
 (gr_line (start 45.908610142288666 56.46864065762139) (end 45.78076118445749 56.58076118445749) (stroke (width .05) (type default))
  (layer "Edge.Cuts"))
 (gr_line (start 45.78076118445749 56.58076118445749) (end 45.668640657621395 56.70861014228866) (stroke (width .05) (type default))
  (layer "Edge.Cuts"))
 (gr_line (start 45.668640657621395 56.70861014228866) (end 45.57416697508023 56.85) (stroke (width .05) (type default)) (layer "Edge.Cuts"))
 (gr_line (start 45.57416697508023 56.85) (end 45.49895660773532 57.002511537925386) (stroke (width .05) (type default)) (layer "Edge.Cuts"))
 (gr_line (start 45.49895660773532 57.002511537925386) (end 45.44429642582421 57.16353524136672) (stroke (width .05) (type default))
  (layer "Edge.Cuts"))
 (gr_line (start 45.44429642582421 57.16353524136672) (end 45.411121680214045 57.330315950113935) (stroke (width .05) (type default))
  (layer "Edge.Cuts"))
 (gr_line (start 45.411121680214045 57.330315950113935) (end 45.4 57.5) (stroke (width .05) (type default)) (layer "Edge.Cuts"))
 (gr_line (start 45.4 57.5) (end 45.411121680214045 57.669684049886065) (stroke (width .05) (type default)) (layer "Edge.Cuts"))
 (gr_line (start 45.411121680214045 57.669684049886065) (end 45.44429642582421 57.83646475863328) (stroke (width .05) (type default))
  (layer "Edge.Cuts"))
 (gr_line (start 45.44429642582421 57.83646475863328) (end 45.49895660773532 57.997488462074614) (stroke (width .05) (type default))
  (layer "Edge.Cuts"))
 (gr_line (start 45.49895660773532 57.997488462074614) (end 45.57416697508023 58.15) (stroke (width .05) (type default)) (layer "Edge.Cuts"))
 (gr_line (start 45.57416697508023 58.15) (end 45.668640657621395 58.29138985771134) (stroke (width .05) (type default)) (layer "Edge.Cuts"))
 (gr_line (start 45.668640657621395 58.29138985771134) (end 45.78076118445749 58.41923881554251) (stroke (width .05) (type default))
  (layer "Edge.Cuts"))
 (gr_line (start 45.78076118445749 58.41923881554251) (end 45.908610142288666 58.53135934237861) (stroke (width .05) (type default))
  (layer "Edge.Cuts"))
 (gr_line (start 45.908610142288666 58.53135934237861) (end 46.05 58.62583302491977) (stroke (width .05) (type default)) (layer "Edge.Cuts"))
 (gr_line (start 46.05 58.62583302491977) (end 46.20251153792538 58.70104339226467) (stroke (width .05) (type default)) (layer "Edge.Cuts"))
 (gr_line (start 46.20251153792538 58.70104339226467) (end 46.363535241366726 58.75570357417579) (stroke (width .05) (type default))
  (layer "Edge.Cuts"))
 (gr_line (start 46.363535241366726 58.75570357417579) (end 46.53031595011393 58.78887831978595) (stroke (width .05) (type default))
  (layer "Edge.Cuts"))
 (gr_line (start 46.53031595011393 58.78887831978595) (end 46.7 58.8) (stroke (width .05) (type default)) (layer "Edge.Cuts"))
 (gr_line (start 46.7 58.8) (end 47.869236616410625 58.8) (stroke (width .05) (type default)) (layer "Edge.Cuts"))
 (gr_line (start 47.869236616410625 58.8) (end 47.99935332123422 58.999137374206725) (stroke (width .05) (type default)) (layer "Edge.Cuts"))
 (gr_line (start 47.99935332123422 58.999137374206725) (end 48.20815631768343 59.243357742444786) (stroke (width .05) (type default))
  (layer "Edge.Cuts"))
 (gr_line (start 48.20815631768343 59.243357742444786) (end 48.44655835836122 59.45877999428793) (stroke (width .05) (type default))
  (layer "Edge.Cuts"))
 (gr_line (start 48.44655835836122 59.45877999428793) (end 48.71062133604549 59.641845620239444) (stroke (width .05) (type default))
  (layer "Edge.Cuts"))
 (gr_line (start 48.71062133604549 59.641845620239444) (end 48.99598325653288 59.78953060229333) (stroke (width .05) (type default))
  (layer "Edge.Cuts"))
 (gr_line (start 48.99598325653288 59.78953060229333) (end 49.29793029339476 59.89939536697628) (stroke (width .05) (type default))
  (layer "Edge.Cuts"))
 (gr_line (start 49.29793029339476 59.89939536697628) (end 49.61147465456702 59.9696250840879) (stroke (width .05) (type default))
  (layer "Edge.Cuts"))
 (gr_line (start 49.61147465456702 59.9696250840879) (end 49.93143697451376 59.9990596454539) (stroke (width .05) (type default))
  (layer "Edge.Cuts"))
 (gr_line (start 49.93143697451376 59.9990596454539) (end 50.25253187094796 59.98721282848001) (stroke (width .05) (type default))
  (layer "Edge.Cuts"))
 (gr_line (start 50.25253187094796 59.98721282848001) (end 50.569455252818095 59.93428032794867) (stroke (width .05) (type default))
  (layer "Edge.Cuts"))
 (gr_line (start 50.569455252818095 59.93428032794867) (end 50.8769719373403 59.84113652338295) (stroke (width .05) (type default))
  (layer "Edge.Cuts"))
 (gr_line (start 50.8769719373403 59.84113652338295) (end 51.170002128751115 59.70932003537692) (stroke (width .05) (type default))
  (layer "Edge.Cuts"))
 (gr_line (start 51.170002128751115 59.70932003537692) (end 51.443705330258624 59.54100830948403) (stroke (width .05) (type default))
  (layer "Edge.Cuts"))
 (gr_line (start 51.443705330258624 59.54100830948403) (end 51.69356030307014 59.338981647506294) (stroke (width .05) (type default))
  (layer "Edge.Cuts"))
 (gr_line (start 51.69356030307014 59.338981647506294) (end 51.915439751672125 59.106577280342975) (stroke (width .05) (type default))
  (layer "Edge.Cuts"))
 (gr_line (start 51.915439751672125 59.106577280342975) (end 52.10567850165378 58.847634241058415) (stroke (width .05) (type default))
  (layer "Edge.Cuts"))
 (gr_line (start 52.10567850165378 58.847634241058415) (end 52.13616441593116 58.8) (stroke (width .05) (type default)) (layer "Edge.Cuts"))
 (gr_line (start 52.13616441593116 58.8) (end 53.3 58.8) (stroke (width .05) (type default)) (layer "Edge.Cuts"))
 (gr_line (start 53.3 58.8) (end 53.46968404988607 58.78887831978595) (stroke (width .05) (type default)) (layer "Edge.Cuts"))
 (gr_line (start 53.46968404988607 58.78887831978595) (end 53.636464758633274 58.75570357417579) (stroke (width .05) (type default))
  (layer "Edge.Cuts"))
 (gr_line (start 53.636464758633274 58.75570357417579) (end 53.79748846207462 58.70104339226467) (stroke (width .05) (type default))
  (layer "Edge.Cuts"))
 (gr_line (start 53.79748846207462 58.70104339226467) (end 53.95 58.62583302491977) (stroke (width .05) (type default)) (layer "Edge.Cuts"))
 (gr_line (start 53.95 58.62583302491977) (end 54.091389857711334 58.53135934237861) (stroke (width .05) (type default)) (layer "Edge.Cuts"))
 (gr_line (start 54.091389857711334 58.53135934237861) (end 54.21923881554251 58.41923881554251) (stroke (width .05) (type default))
  (layer "Edge.Cuts"))
 (gr_line (start 54.21923881554251 58.41923881554251) (end 54.331359342378605 58.29138985771134) (stroke (width .05) (type default))
  (layer "Edge.Cuts"))
 (gr_line (start 54.331359342378605 58.29138985771134) (end 54.42583302491977 58.15) (stroke (width .05) (type default)) (layer "Edge.Cuts"))
 (gr_line (start 54.42583302491977 58.15) (end 54.50104339226467 57.997488462074614) (stroke (width .05) (type default)) (layer "Edge.Cuts"))
 (gr_line (start 54.50104339226467 57.997488462074614) (end 54.55570357417579 57.83646475863328) (stroke (width .05) (type default))
  (layer "Edge.Cuts"))
 (gr_line (start 54.55570357417579 57.83646475863328) (end 54.588878319785955 57.669684049886065) (stroke (width .05) (type default))
  (layer "Edge.Cuts"))
 (gr_line (start 54.588878319785955 57.669684049886065) (end 54.6 57.5) (stroke (width .05) (type default)) (layer "Edge.Cuts"))
 (gr_line (start 54.6 57.5) (end 54.588878319785955 57.330315950113935) (stroke (width .05) (type default)) (layer "Edge.Cuts"))
 (gr_line (start 54.588878319785955 57.330315950113935) (end 54.55570357417579 57.16353524136672) (stroke (width .05) (type default))
  (layer "Edge.Cuts"))
 (gr_line (start 54.55570357417579 57.16353524136672) (end 54.50104339226468 57.002511537925386) (stroke (width .05) (type default))
  (layer "Edge.Cuts"))
 (gr_line (start 54.50104339226468 57.002511537925386) (end 54.42583302491977 56.85) (stroke (width .05) (type default)) (layer "Edge.Cuts"))
 (gr_line (start 54.42583302491977 56.85) (end 54.331359342378605 56.70861014228866) (stroke (width .05) (type default)) (layer "Edge.Cuts"))
 (gr_line (start 54.331359342378605 56.70861014228866) (end 54.21923881554251 56.58076118445749) (stroke (width .05) (type default))
  (layer "Edge.Cuts"))
 (gr_line (start 54.21923881554251 56.58076118445749) (end 54.091389857711334 56.46864065762139) (stroke (width .05) (type default))
  (layer "Edge.Cuts"))
 (gr_line (start 54.091389857711334 56.46864065762139) (end 53.95 56.37416697508023) (stroke (width .05) (type default)) (layer "Edge.Cuts"))
 (gr_line (start 53.95 56.37416697508023) (end 53.79748846207462 56.29895660773533) (stroke (width .05) (type default)) (layer "Edge.Cuts"))
 (gr_line (start 53.79748846207462 56.29895660773533) (end 53.747657910476015 56.28204141477367) (stroke (width .05) (type default))
  (layer "Edge.Cuts"))
 (gr_line (start 53.747657910476015 56.28204141477367) (end 56.90567850165378 51.347634241058415) (stroke (width .05) (type default))
  (layer "Edge.Cuts"))
 (gr_line (start 56.90567850165378 51.347634241058415) (end 57.05888963109352 51.071175818686264) (stroke (width .05) (type default))
  (layer "Edge.Cuts"))
 (gr_line (start 57.05888963109352 51.071175818686264) (end 57.175993617117086 50.777595223377084) (stroke (width .05) (type default))
  (layer "Edge.Cuts"))
 (gr_line (start 57.175993617117086 50.777595223377084) (end 57.25511861509793 50.47158518403322) (stroke (width .05) (type default))
  (layer "Edge.Cuts"))
 (gr_line (start 57.25511861509793 50.47158518403322) (end 57.29499985423423 50.15803710757659) (stroke (width .05) (type default))
  (layer "Edge.Cuts"))
 (gr_line (start 57.29499985423423 50.15803710757659) (end 57.29499985423423 49.84196289242341) (stroke (width .05) (type default))
  (layer "Edge.Cuts"))
 (gr_line (start 57.29499985423423 49.84196289242341) (end 57.25511861509793 49.52841481596678) (stroke (width .05) (type default))
  (layer "Edge.Cuts"))
 (gr_line (start 57.25511861509793 49.52841481596678) (end 57.175993617117086 49.222404776622916) (stroke (width .05) (type default))
  (layer "Edge.Cuts"))
 (gr_line (start 57.175993617117086 49.222404776622916) (end 57.05888963109352 48.928824181313736) (stroke (width .05) (type default))
  (layer "Edge.Cuts"))
 (gr_line (start 57.05888963109352 48.928824181313736) (end 56.90567850165378 48.652365758941585) (stroke (width .05) (type default))
  (layer "Edge.Cuts"))
 (gr_line (start 56.90567850165378 48.652365758941585) (end 52.10567850165378 41.152365758941585) (stroke (width .05) (type default))
  (layer "Edge.Cuts"))
 (gr_line (start 52.10567850165378 41.152365758941585) (end 51.915439751672125 40.893422719657025) (stroke (width .05) (type default))
  (layer "Edge.Cuts"))
 (gr_line (start 51.915439751672125 40.893422719657025) (end 51.69356030307014 40.661018352493706) (stroke (width .05) (type default))
  (layer "Edge.Cuts")))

